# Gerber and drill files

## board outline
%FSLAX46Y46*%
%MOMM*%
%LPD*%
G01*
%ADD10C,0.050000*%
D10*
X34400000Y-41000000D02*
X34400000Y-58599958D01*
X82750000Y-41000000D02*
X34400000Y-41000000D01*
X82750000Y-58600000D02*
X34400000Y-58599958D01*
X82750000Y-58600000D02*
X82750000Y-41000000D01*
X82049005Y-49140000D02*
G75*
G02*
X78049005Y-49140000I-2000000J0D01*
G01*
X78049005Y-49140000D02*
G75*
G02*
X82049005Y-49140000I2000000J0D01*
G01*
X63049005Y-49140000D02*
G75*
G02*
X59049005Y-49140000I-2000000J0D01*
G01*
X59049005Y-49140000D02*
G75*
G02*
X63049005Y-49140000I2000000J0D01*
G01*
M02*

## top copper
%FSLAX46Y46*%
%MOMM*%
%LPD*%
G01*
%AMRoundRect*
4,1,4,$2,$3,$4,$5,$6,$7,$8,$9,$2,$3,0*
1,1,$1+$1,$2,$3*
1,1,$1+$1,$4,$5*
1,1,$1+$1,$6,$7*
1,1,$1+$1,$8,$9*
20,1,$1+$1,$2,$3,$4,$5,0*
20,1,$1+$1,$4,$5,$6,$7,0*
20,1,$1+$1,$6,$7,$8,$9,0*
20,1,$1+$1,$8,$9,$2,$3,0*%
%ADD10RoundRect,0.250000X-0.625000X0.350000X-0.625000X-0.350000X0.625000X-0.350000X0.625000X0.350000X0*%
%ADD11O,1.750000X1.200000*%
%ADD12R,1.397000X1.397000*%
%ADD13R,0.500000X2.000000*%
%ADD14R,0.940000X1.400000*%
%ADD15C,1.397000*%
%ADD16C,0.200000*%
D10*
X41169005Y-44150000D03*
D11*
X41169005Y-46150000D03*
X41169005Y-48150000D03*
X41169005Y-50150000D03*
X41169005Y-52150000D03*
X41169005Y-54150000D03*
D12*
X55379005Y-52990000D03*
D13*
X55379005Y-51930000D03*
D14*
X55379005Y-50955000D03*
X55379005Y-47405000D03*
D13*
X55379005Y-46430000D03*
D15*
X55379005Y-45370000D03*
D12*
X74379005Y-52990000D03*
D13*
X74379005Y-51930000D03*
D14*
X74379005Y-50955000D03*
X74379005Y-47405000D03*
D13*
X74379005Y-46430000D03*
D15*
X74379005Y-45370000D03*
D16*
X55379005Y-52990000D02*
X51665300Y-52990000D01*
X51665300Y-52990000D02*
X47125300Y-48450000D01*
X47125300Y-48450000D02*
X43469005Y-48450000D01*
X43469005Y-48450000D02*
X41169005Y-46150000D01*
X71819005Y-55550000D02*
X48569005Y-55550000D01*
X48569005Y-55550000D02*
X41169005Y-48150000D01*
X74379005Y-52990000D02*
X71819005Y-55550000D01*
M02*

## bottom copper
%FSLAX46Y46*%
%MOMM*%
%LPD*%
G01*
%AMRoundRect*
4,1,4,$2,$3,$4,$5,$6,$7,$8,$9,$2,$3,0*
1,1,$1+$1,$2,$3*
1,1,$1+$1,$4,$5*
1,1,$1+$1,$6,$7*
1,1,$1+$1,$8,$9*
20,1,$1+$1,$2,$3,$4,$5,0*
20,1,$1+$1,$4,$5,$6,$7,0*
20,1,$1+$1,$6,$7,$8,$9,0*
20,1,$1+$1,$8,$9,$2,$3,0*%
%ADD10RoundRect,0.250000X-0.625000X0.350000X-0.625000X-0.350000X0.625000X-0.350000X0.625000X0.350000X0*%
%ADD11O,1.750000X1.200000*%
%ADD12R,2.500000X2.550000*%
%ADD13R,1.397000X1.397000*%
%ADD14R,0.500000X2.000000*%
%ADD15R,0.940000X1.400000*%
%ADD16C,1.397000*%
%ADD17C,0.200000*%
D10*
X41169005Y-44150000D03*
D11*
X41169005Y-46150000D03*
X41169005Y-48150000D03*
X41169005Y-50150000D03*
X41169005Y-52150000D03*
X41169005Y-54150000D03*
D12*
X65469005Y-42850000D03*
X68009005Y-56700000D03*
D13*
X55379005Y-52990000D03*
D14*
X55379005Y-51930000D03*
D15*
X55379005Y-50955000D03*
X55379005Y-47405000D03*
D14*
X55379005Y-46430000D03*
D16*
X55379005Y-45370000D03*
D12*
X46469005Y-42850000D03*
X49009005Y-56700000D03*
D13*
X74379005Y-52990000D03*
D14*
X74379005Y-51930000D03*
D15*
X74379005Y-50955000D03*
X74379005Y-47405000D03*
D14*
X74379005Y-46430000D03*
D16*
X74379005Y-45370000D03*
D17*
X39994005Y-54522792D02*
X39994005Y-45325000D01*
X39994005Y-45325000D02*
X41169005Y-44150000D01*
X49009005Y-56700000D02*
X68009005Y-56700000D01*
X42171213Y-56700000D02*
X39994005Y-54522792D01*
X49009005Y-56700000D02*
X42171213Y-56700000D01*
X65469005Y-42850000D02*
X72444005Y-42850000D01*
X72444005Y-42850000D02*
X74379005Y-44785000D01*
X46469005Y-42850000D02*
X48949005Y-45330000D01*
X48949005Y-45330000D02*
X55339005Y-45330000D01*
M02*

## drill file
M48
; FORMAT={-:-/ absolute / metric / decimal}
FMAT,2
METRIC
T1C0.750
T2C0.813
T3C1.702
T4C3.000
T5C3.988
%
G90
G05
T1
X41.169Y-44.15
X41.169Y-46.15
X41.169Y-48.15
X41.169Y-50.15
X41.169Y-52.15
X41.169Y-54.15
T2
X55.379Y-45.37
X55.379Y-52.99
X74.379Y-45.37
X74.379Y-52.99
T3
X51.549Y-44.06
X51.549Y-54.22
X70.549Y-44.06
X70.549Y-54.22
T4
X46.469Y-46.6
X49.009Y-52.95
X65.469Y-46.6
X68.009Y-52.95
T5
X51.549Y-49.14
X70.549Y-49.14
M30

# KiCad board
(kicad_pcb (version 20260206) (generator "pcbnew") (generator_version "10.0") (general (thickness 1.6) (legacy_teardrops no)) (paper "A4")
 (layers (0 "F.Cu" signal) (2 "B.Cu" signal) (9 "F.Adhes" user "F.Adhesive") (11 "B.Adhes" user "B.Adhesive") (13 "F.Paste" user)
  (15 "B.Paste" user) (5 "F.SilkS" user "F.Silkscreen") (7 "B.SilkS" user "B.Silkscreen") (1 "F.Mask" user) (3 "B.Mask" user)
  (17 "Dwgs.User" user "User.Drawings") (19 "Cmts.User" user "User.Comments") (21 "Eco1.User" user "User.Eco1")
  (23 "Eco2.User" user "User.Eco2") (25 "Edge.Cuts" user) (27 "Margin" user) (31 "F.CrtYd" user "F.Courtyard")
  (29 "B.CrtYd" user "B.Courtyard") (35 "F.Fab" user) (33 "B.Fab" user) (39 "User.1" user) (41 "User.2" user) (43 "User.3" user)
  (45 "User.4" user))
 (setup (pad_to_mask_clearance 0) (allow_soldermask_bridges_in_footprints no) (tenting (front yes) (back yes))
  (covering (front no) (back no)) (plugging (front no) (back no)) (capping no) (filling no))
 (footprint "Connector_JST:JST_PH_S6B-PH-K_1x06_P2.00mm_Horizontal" (layer "F.Cu") (at 41.169005 44.15 -90)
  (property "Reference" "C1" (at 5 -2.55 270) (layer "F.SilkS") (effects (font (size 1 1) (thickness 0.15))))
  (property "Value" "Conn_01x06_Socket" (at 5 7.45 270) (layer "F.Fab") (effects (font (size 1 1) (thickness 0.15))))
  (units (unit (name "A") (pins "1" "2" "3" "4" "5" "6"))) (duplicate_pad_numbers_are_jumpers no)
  (pad "1" thru_hole roundrect (at 0 0 270) (size 1.2 1.75) (drill 0.75) (layers "*.Cu" "*.Mask") (remove_unused_layers no)
   (roundrect_rratio 0.208333) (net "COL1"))
  (pad "2" thru_hole oval (at 2 0 270) (size 1.2 1.75) (drill 0.75) (layers "*.Cu" "*.Mask") (remove_unused_layers no) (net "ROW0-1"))
  (pad "3" thru_hole oval (at 4 0 270) (size 1.2 1.75) (drill 0.75) (layers "*.Cu" "*.Mask") (remove_unused_layers no) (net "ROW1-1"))
  (pad "4" thru_hole oval (at 6 0 270) (size 1.2 1.75) (drill 0.75) (layers "*.Cu" "*.Mask") (remove_unused_layers no) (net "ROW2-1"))
  (pad "5" thru_hole oval (at 8 0 270) (size 1.2 1.75) (drill 0.75) (layers "*.Cu" "*.Mask") (remove_unused_layers no) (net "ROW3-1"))
  (pad "6" thru_hole oval (at 10 0 270) (size 1.2 1.75) (drill 0.75) (layers "*.Cu" "*.Mask") (remove_unused_layers no) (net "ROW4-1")))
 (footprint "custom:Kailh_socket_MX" (layer "F.Cu") (at 70.549005 49.14 90)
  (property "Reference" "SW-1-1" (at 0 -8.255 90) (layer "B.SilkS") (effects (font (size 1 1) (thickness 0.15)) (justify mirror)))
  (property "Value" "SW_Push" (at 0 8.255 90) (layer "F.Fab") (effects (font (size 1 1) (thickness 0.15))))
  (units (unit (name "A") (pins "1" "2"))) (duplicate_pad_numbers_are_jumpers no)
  (pad "" np_thru_hole circle (at -5.08 0 90) (size 1.7018 1.7018) (drill 1.7018) (layers "*.Cu" "*.Mask"))
  (pad "" np_thru_hole circle (at -3.81 -2.54 90) (size 3 3) (drill 3) (layers "*.Cu" "*.Mask"))
  (pad "" np_thru_hole circle (at 0 0 90) (size 3.9878 3.9878) (drill 3.9878) (layers "*.Cu" "*.Mask"))
  (pad "" np_thru_hole circle (at 2.54 -5.08 90) (size 3 3) (drill 3) (layers "*.Cu" "*.Mask"))
  (pad "" np_thru_hole circle (at 5.08 0 90) (size 1.7018 1.7018) (drill 1.7018) (layers "*.Cu" "*.Mask"))
  (pad "1" smd rect (at 6.29 -5.08 90) (size 2.55 2.5) (layers "B.Cu" "B.Mask" "B.Paste") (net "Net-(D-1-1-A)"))
  (pad "2" smd rect (at -7.56 -2.54 90) (size 2.55 2.5) (layers "B.Cu" "B.Mask" "B.Paste") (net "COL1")))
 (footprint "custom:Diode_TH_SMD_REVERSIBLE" (layer "F.Cu") (at 55.379005 49.18 90)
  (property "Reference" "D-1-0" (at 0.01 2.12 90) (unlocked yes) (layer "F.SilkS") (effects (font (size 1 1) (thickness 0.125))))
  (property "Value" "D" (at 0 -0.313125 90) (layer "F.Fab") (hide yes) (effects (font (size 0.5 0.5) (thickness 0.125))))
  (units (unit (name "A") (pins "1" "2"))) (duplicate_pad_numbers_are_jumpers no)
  (pad "1" thru_hole rect (at -3.81 0 90) (size 1.397 1.397) (drill 0.8128) (layers "*.Cu" "*.Mask") (remove_unused_layers no)
   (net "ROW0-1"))
  (pad "1" smd rect (at -2.75 0 270) (size 2 0.5) (layers "F.Cu") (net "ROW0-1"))
  (pad "1" smd rect (at -2.75 0 90) (size 2 0.5) (layers "B.Cu") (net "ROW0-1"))
  (pad "1" smd rect (at -1.775 0 270) (size 1.4 0.94) (layers "F.Cu" "F.Mask" "F.Paste") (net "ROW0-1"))
  (pad "1" smd rect (at -1.775 0 90) (size 1.4 0.94) (layers "B.Cu" "B.Mask" "B.Paste") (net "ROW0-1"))
  (pad "2" smd rect (at 1.775 0 270) (size 1.4 0.94) (layers "F.Cu" "F.Mask" "F.Paste") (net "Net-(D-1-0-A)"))
  (pad "2" smd rect (at 1.775 0 90) (size 1.4 0.94) (layers "B.Cu" "B.Mask" "B.Paste") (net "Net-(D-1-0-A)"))
  (pad "2" smd rect (at 2.75 0 270) (size 2 0.5) (layers "F.Cu") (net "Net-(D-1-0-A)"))
  (pad "2" smd rect (at 2.75 0 90) (size 2 0.5) (layers "B.Cu") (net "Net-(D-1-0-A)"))
  (pad "2" thru_hole circle (at 3.81 0 90) (size 1.397 1.397) (drill 0.8128) (layers "*.Cu" "*.Mask") (remove_unused_layers no)
   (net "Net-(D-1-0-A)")))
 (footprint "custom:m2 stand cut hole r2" (layer "F.Cu") (at 80.049005 49.14 90)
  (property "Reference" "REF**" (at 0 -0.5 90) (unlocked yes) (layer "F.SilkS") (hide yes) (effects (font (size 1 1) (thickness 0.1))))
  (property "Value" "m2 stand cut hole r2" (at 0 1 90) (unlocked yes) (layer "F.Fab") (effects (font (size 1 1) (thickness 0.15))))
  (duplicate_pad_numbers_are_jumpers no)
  (fp_circle (center 0 0) (end 2 0) (stroke (width 0.05) (type default)) (fill no) (layer "Edge.Cuts")))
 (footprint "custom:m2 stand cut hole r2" (layer "F.Cu") (at 61.049005 49.14 90)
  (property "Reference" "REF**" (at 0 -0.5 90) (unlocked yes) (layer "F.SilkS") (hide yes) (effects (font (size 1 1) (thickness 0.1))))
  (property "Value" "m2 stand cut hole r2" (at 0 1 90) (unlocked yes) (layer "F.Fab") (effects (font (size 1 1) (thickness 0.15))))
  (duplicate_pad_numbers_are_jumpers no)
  (fp_circle (center 0 0) (end 2 0) (stroke (width 0.05) (type default)) (fill no) (layer "Edge.Cuts")))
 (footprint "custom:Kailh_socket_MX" (layer "F.Cu") (at 51.549005 49.14 90)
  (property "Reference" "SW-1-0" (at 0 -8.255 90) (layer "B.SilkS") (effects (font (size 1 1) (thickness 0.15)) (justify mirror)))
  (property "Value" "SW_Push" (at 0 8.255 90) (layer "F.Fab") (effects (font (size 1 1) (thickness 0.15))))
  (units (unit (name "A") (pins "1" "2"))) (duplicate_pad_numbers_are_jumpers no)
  (pad "" np_thru_hole circle (at -5.08 0 90) (size 1.7018 1.7018) (drill 1.7018) (layers "*.Cu" "*.Mask"))
  (pad "" np_thru_hole circle (at -3.81 -2.54 90) (size 3 3) (drill 3) (layers "*.Cu" "*.Mask"))
  (pad "" np_thru_hole circle (at 0 0 90) (size 3.9878 3.9878) (drill 3.9878) (layers "*.Cu" "*.Mask"))
  (pad "" np_thru_hole circle (at 2.54 -5.08 90) (size 3 3) (drill 3) (layers "*.Cu" "*.Mask"))
  (pad "" np_thru_hole circle (at 5.08 0 90) (size 1.7018 1.7018) (drill 1.7018) (layers "*.Cu" "*.Mask"))
  (pad "1" smd rect (at 6.29 -5.08 90) (size 2.55 2.5) (layers "B.Cu" "B.Mask" "B.Paste") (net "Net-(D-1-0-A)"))
  (pad "2" smd rect (at -7.56 -2.54 90) (size 2.55 2.5) (layers "B.Cu" "B.Mask" "B.Paste") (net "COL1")))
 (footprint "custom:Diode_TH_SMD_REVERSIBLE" (layer "F.Cu") (at 74.379005 49.18 90)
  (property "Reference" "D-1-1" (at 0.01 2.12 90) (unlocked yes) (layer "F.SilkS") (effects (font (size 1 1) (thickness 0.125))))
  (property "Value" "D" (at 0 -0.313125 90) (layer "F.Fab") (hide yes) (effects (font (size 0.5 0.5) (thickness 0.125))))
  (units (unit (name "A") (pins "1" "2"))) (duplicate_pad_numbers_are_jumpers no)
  (pad "1" thru_hole rect (at -3.81 0 90) (size 1.397 1.397) (drill 0.8128) (layers "*.Cu" "*.Mask") (remove_unused_layers no)
   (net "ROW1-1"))
  (pad "1" smd rect (at -2.75 0 270) (size 2 0.5) (layers "F.Cu") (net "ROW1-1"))
  (pad "1" smd rect (at -2.75 0 90) (size 2 0.5) (layers "B.Cu") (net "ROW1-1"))
  (pad "1" smd rect (at -1.775 0 270) (size 1.4 0.94) (layers "F.Cu" "F.Mask" "F.Paste") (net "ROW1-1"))
  (pad "1" smd rect (at -1.775 0 90) (size 1.4 0.94) (layers "B.Cu" "B.Mask" "B.Paste") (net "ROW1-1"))
  (pad "2" smd rect (at 1.775 0 270) (size 1.4 0.94) (layers "F.Cu" "F.Mask" "F.Paste") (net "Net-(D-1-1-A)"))
  (pad "2" smd rect (at 1.775 0 90) (size 1.4 0.94) (layers "B.Cu" "B.Mask" "B.Paste") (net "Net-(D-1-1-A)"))
  (pad "2" smd rect (at 2.75 0 270) (size 2 0.5) (layers "F.Cu") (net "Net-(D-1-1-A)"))
  (pad "2" smd rect (at 2.75 0 90) (size 2 0.5) (layers "B.Cu") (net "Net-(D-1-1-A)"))
  (pad "2" thru_hole circle (at 3.81 0 90) (size 1.397 1.397) (drill 0.8128) (layers "*.Cu" "*.Mask") (remove_unused_layers no)
   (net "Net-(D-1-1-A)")))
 (gr_line (start 34.4 41) (end 34.4 58.599958) (stroke (width 0.05) (type default)) (layer "Edge.Cuts"))
 (gr_line (start 82.75 41) (end 34.4 41) (stroke (width 0.05) (type default)) (layer "Edge.Cuts"))
 (gr_line (start 82.75 58.6) (end 34.4 58.599958) (stroke (width 0.05) (type default)) (layer "Edge.Cuts"))
 (gr_line (start 82.75 58.6) (end 82.75 41) (stroke (width 0.05) (type default)) (layer "Edge.Cuts"))
 (segment (start 39.994005 54.522792) (end 39.994005 45.325) (width 0.2) (layer "B.Cu") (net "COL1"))
 (segment (start 39.994005 45.325) (end 41.169005 44.15) (width 0.2) (layer "B.Cu") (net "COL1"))
 (segment (start 49.009005 56.7) (end 68.009005 56.7) (width 0.2) (layer "B.Cu") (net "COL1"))
 (segment (start 42.171213 56.7) (end 39.994005 54.522792) (width 0.2) (layer "B.Cu") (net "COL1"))
 (segment (start 49.009005 56.7) (end 42.171213 56.7) (width 0.2) (layer "B.Cu") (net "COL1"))
 (segment (start 55.379005 52.99) (end 51.6653 52.99) (width 0.2) (layer "F.Cu") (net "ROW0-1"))
 (segment (start 51.6653 52.99) (end 47.1253 48.45) (width 0.2) (layer "F.Cu") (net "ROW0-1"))
 (segment (start 47.1253 48.45) (end 43.469005 48.45) (width 0.2) (layer "F.Cu") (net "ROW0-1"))
 (segment (start 43.469005 48.45) (end 41.169005 46.15) (width 0.2) (layer "F.Cu") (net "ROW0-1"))
 (segment (start 71.819005 55.55) (end 48.569005 55.55) (width 0.2) (layer "F.Cu") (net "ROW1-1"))
 (segment (start 48.569005 55.55) (end 41.169005 48.15) (width 0.2) (layer "F.Cu") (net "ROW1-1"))
 (segment (start 74.379005 52.99) (end 71.819005 55.55) (width 0.2) (layer "F.Cu") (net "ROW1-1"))
 (segment (start 65.469005 42.85) (end 72.444005 42.85) (width 0.2) (layer "B.Cu") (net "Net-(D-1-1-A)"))
 (segment (start 72.444005 42.85) (end 74.379005 44.785) (width 0.2) (layer "B.Cu") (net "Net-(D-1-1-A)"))
 (segment (start 46.469005 42.85) (end 48.949005 45.33) (width 0.2) (layer "B.Cu") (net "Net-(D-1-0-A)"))
 (segment (start 48.949005 45.33) (end 55.339005 45.33) (width 0.2) (layer "B.Cu") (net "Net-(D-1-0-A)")))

